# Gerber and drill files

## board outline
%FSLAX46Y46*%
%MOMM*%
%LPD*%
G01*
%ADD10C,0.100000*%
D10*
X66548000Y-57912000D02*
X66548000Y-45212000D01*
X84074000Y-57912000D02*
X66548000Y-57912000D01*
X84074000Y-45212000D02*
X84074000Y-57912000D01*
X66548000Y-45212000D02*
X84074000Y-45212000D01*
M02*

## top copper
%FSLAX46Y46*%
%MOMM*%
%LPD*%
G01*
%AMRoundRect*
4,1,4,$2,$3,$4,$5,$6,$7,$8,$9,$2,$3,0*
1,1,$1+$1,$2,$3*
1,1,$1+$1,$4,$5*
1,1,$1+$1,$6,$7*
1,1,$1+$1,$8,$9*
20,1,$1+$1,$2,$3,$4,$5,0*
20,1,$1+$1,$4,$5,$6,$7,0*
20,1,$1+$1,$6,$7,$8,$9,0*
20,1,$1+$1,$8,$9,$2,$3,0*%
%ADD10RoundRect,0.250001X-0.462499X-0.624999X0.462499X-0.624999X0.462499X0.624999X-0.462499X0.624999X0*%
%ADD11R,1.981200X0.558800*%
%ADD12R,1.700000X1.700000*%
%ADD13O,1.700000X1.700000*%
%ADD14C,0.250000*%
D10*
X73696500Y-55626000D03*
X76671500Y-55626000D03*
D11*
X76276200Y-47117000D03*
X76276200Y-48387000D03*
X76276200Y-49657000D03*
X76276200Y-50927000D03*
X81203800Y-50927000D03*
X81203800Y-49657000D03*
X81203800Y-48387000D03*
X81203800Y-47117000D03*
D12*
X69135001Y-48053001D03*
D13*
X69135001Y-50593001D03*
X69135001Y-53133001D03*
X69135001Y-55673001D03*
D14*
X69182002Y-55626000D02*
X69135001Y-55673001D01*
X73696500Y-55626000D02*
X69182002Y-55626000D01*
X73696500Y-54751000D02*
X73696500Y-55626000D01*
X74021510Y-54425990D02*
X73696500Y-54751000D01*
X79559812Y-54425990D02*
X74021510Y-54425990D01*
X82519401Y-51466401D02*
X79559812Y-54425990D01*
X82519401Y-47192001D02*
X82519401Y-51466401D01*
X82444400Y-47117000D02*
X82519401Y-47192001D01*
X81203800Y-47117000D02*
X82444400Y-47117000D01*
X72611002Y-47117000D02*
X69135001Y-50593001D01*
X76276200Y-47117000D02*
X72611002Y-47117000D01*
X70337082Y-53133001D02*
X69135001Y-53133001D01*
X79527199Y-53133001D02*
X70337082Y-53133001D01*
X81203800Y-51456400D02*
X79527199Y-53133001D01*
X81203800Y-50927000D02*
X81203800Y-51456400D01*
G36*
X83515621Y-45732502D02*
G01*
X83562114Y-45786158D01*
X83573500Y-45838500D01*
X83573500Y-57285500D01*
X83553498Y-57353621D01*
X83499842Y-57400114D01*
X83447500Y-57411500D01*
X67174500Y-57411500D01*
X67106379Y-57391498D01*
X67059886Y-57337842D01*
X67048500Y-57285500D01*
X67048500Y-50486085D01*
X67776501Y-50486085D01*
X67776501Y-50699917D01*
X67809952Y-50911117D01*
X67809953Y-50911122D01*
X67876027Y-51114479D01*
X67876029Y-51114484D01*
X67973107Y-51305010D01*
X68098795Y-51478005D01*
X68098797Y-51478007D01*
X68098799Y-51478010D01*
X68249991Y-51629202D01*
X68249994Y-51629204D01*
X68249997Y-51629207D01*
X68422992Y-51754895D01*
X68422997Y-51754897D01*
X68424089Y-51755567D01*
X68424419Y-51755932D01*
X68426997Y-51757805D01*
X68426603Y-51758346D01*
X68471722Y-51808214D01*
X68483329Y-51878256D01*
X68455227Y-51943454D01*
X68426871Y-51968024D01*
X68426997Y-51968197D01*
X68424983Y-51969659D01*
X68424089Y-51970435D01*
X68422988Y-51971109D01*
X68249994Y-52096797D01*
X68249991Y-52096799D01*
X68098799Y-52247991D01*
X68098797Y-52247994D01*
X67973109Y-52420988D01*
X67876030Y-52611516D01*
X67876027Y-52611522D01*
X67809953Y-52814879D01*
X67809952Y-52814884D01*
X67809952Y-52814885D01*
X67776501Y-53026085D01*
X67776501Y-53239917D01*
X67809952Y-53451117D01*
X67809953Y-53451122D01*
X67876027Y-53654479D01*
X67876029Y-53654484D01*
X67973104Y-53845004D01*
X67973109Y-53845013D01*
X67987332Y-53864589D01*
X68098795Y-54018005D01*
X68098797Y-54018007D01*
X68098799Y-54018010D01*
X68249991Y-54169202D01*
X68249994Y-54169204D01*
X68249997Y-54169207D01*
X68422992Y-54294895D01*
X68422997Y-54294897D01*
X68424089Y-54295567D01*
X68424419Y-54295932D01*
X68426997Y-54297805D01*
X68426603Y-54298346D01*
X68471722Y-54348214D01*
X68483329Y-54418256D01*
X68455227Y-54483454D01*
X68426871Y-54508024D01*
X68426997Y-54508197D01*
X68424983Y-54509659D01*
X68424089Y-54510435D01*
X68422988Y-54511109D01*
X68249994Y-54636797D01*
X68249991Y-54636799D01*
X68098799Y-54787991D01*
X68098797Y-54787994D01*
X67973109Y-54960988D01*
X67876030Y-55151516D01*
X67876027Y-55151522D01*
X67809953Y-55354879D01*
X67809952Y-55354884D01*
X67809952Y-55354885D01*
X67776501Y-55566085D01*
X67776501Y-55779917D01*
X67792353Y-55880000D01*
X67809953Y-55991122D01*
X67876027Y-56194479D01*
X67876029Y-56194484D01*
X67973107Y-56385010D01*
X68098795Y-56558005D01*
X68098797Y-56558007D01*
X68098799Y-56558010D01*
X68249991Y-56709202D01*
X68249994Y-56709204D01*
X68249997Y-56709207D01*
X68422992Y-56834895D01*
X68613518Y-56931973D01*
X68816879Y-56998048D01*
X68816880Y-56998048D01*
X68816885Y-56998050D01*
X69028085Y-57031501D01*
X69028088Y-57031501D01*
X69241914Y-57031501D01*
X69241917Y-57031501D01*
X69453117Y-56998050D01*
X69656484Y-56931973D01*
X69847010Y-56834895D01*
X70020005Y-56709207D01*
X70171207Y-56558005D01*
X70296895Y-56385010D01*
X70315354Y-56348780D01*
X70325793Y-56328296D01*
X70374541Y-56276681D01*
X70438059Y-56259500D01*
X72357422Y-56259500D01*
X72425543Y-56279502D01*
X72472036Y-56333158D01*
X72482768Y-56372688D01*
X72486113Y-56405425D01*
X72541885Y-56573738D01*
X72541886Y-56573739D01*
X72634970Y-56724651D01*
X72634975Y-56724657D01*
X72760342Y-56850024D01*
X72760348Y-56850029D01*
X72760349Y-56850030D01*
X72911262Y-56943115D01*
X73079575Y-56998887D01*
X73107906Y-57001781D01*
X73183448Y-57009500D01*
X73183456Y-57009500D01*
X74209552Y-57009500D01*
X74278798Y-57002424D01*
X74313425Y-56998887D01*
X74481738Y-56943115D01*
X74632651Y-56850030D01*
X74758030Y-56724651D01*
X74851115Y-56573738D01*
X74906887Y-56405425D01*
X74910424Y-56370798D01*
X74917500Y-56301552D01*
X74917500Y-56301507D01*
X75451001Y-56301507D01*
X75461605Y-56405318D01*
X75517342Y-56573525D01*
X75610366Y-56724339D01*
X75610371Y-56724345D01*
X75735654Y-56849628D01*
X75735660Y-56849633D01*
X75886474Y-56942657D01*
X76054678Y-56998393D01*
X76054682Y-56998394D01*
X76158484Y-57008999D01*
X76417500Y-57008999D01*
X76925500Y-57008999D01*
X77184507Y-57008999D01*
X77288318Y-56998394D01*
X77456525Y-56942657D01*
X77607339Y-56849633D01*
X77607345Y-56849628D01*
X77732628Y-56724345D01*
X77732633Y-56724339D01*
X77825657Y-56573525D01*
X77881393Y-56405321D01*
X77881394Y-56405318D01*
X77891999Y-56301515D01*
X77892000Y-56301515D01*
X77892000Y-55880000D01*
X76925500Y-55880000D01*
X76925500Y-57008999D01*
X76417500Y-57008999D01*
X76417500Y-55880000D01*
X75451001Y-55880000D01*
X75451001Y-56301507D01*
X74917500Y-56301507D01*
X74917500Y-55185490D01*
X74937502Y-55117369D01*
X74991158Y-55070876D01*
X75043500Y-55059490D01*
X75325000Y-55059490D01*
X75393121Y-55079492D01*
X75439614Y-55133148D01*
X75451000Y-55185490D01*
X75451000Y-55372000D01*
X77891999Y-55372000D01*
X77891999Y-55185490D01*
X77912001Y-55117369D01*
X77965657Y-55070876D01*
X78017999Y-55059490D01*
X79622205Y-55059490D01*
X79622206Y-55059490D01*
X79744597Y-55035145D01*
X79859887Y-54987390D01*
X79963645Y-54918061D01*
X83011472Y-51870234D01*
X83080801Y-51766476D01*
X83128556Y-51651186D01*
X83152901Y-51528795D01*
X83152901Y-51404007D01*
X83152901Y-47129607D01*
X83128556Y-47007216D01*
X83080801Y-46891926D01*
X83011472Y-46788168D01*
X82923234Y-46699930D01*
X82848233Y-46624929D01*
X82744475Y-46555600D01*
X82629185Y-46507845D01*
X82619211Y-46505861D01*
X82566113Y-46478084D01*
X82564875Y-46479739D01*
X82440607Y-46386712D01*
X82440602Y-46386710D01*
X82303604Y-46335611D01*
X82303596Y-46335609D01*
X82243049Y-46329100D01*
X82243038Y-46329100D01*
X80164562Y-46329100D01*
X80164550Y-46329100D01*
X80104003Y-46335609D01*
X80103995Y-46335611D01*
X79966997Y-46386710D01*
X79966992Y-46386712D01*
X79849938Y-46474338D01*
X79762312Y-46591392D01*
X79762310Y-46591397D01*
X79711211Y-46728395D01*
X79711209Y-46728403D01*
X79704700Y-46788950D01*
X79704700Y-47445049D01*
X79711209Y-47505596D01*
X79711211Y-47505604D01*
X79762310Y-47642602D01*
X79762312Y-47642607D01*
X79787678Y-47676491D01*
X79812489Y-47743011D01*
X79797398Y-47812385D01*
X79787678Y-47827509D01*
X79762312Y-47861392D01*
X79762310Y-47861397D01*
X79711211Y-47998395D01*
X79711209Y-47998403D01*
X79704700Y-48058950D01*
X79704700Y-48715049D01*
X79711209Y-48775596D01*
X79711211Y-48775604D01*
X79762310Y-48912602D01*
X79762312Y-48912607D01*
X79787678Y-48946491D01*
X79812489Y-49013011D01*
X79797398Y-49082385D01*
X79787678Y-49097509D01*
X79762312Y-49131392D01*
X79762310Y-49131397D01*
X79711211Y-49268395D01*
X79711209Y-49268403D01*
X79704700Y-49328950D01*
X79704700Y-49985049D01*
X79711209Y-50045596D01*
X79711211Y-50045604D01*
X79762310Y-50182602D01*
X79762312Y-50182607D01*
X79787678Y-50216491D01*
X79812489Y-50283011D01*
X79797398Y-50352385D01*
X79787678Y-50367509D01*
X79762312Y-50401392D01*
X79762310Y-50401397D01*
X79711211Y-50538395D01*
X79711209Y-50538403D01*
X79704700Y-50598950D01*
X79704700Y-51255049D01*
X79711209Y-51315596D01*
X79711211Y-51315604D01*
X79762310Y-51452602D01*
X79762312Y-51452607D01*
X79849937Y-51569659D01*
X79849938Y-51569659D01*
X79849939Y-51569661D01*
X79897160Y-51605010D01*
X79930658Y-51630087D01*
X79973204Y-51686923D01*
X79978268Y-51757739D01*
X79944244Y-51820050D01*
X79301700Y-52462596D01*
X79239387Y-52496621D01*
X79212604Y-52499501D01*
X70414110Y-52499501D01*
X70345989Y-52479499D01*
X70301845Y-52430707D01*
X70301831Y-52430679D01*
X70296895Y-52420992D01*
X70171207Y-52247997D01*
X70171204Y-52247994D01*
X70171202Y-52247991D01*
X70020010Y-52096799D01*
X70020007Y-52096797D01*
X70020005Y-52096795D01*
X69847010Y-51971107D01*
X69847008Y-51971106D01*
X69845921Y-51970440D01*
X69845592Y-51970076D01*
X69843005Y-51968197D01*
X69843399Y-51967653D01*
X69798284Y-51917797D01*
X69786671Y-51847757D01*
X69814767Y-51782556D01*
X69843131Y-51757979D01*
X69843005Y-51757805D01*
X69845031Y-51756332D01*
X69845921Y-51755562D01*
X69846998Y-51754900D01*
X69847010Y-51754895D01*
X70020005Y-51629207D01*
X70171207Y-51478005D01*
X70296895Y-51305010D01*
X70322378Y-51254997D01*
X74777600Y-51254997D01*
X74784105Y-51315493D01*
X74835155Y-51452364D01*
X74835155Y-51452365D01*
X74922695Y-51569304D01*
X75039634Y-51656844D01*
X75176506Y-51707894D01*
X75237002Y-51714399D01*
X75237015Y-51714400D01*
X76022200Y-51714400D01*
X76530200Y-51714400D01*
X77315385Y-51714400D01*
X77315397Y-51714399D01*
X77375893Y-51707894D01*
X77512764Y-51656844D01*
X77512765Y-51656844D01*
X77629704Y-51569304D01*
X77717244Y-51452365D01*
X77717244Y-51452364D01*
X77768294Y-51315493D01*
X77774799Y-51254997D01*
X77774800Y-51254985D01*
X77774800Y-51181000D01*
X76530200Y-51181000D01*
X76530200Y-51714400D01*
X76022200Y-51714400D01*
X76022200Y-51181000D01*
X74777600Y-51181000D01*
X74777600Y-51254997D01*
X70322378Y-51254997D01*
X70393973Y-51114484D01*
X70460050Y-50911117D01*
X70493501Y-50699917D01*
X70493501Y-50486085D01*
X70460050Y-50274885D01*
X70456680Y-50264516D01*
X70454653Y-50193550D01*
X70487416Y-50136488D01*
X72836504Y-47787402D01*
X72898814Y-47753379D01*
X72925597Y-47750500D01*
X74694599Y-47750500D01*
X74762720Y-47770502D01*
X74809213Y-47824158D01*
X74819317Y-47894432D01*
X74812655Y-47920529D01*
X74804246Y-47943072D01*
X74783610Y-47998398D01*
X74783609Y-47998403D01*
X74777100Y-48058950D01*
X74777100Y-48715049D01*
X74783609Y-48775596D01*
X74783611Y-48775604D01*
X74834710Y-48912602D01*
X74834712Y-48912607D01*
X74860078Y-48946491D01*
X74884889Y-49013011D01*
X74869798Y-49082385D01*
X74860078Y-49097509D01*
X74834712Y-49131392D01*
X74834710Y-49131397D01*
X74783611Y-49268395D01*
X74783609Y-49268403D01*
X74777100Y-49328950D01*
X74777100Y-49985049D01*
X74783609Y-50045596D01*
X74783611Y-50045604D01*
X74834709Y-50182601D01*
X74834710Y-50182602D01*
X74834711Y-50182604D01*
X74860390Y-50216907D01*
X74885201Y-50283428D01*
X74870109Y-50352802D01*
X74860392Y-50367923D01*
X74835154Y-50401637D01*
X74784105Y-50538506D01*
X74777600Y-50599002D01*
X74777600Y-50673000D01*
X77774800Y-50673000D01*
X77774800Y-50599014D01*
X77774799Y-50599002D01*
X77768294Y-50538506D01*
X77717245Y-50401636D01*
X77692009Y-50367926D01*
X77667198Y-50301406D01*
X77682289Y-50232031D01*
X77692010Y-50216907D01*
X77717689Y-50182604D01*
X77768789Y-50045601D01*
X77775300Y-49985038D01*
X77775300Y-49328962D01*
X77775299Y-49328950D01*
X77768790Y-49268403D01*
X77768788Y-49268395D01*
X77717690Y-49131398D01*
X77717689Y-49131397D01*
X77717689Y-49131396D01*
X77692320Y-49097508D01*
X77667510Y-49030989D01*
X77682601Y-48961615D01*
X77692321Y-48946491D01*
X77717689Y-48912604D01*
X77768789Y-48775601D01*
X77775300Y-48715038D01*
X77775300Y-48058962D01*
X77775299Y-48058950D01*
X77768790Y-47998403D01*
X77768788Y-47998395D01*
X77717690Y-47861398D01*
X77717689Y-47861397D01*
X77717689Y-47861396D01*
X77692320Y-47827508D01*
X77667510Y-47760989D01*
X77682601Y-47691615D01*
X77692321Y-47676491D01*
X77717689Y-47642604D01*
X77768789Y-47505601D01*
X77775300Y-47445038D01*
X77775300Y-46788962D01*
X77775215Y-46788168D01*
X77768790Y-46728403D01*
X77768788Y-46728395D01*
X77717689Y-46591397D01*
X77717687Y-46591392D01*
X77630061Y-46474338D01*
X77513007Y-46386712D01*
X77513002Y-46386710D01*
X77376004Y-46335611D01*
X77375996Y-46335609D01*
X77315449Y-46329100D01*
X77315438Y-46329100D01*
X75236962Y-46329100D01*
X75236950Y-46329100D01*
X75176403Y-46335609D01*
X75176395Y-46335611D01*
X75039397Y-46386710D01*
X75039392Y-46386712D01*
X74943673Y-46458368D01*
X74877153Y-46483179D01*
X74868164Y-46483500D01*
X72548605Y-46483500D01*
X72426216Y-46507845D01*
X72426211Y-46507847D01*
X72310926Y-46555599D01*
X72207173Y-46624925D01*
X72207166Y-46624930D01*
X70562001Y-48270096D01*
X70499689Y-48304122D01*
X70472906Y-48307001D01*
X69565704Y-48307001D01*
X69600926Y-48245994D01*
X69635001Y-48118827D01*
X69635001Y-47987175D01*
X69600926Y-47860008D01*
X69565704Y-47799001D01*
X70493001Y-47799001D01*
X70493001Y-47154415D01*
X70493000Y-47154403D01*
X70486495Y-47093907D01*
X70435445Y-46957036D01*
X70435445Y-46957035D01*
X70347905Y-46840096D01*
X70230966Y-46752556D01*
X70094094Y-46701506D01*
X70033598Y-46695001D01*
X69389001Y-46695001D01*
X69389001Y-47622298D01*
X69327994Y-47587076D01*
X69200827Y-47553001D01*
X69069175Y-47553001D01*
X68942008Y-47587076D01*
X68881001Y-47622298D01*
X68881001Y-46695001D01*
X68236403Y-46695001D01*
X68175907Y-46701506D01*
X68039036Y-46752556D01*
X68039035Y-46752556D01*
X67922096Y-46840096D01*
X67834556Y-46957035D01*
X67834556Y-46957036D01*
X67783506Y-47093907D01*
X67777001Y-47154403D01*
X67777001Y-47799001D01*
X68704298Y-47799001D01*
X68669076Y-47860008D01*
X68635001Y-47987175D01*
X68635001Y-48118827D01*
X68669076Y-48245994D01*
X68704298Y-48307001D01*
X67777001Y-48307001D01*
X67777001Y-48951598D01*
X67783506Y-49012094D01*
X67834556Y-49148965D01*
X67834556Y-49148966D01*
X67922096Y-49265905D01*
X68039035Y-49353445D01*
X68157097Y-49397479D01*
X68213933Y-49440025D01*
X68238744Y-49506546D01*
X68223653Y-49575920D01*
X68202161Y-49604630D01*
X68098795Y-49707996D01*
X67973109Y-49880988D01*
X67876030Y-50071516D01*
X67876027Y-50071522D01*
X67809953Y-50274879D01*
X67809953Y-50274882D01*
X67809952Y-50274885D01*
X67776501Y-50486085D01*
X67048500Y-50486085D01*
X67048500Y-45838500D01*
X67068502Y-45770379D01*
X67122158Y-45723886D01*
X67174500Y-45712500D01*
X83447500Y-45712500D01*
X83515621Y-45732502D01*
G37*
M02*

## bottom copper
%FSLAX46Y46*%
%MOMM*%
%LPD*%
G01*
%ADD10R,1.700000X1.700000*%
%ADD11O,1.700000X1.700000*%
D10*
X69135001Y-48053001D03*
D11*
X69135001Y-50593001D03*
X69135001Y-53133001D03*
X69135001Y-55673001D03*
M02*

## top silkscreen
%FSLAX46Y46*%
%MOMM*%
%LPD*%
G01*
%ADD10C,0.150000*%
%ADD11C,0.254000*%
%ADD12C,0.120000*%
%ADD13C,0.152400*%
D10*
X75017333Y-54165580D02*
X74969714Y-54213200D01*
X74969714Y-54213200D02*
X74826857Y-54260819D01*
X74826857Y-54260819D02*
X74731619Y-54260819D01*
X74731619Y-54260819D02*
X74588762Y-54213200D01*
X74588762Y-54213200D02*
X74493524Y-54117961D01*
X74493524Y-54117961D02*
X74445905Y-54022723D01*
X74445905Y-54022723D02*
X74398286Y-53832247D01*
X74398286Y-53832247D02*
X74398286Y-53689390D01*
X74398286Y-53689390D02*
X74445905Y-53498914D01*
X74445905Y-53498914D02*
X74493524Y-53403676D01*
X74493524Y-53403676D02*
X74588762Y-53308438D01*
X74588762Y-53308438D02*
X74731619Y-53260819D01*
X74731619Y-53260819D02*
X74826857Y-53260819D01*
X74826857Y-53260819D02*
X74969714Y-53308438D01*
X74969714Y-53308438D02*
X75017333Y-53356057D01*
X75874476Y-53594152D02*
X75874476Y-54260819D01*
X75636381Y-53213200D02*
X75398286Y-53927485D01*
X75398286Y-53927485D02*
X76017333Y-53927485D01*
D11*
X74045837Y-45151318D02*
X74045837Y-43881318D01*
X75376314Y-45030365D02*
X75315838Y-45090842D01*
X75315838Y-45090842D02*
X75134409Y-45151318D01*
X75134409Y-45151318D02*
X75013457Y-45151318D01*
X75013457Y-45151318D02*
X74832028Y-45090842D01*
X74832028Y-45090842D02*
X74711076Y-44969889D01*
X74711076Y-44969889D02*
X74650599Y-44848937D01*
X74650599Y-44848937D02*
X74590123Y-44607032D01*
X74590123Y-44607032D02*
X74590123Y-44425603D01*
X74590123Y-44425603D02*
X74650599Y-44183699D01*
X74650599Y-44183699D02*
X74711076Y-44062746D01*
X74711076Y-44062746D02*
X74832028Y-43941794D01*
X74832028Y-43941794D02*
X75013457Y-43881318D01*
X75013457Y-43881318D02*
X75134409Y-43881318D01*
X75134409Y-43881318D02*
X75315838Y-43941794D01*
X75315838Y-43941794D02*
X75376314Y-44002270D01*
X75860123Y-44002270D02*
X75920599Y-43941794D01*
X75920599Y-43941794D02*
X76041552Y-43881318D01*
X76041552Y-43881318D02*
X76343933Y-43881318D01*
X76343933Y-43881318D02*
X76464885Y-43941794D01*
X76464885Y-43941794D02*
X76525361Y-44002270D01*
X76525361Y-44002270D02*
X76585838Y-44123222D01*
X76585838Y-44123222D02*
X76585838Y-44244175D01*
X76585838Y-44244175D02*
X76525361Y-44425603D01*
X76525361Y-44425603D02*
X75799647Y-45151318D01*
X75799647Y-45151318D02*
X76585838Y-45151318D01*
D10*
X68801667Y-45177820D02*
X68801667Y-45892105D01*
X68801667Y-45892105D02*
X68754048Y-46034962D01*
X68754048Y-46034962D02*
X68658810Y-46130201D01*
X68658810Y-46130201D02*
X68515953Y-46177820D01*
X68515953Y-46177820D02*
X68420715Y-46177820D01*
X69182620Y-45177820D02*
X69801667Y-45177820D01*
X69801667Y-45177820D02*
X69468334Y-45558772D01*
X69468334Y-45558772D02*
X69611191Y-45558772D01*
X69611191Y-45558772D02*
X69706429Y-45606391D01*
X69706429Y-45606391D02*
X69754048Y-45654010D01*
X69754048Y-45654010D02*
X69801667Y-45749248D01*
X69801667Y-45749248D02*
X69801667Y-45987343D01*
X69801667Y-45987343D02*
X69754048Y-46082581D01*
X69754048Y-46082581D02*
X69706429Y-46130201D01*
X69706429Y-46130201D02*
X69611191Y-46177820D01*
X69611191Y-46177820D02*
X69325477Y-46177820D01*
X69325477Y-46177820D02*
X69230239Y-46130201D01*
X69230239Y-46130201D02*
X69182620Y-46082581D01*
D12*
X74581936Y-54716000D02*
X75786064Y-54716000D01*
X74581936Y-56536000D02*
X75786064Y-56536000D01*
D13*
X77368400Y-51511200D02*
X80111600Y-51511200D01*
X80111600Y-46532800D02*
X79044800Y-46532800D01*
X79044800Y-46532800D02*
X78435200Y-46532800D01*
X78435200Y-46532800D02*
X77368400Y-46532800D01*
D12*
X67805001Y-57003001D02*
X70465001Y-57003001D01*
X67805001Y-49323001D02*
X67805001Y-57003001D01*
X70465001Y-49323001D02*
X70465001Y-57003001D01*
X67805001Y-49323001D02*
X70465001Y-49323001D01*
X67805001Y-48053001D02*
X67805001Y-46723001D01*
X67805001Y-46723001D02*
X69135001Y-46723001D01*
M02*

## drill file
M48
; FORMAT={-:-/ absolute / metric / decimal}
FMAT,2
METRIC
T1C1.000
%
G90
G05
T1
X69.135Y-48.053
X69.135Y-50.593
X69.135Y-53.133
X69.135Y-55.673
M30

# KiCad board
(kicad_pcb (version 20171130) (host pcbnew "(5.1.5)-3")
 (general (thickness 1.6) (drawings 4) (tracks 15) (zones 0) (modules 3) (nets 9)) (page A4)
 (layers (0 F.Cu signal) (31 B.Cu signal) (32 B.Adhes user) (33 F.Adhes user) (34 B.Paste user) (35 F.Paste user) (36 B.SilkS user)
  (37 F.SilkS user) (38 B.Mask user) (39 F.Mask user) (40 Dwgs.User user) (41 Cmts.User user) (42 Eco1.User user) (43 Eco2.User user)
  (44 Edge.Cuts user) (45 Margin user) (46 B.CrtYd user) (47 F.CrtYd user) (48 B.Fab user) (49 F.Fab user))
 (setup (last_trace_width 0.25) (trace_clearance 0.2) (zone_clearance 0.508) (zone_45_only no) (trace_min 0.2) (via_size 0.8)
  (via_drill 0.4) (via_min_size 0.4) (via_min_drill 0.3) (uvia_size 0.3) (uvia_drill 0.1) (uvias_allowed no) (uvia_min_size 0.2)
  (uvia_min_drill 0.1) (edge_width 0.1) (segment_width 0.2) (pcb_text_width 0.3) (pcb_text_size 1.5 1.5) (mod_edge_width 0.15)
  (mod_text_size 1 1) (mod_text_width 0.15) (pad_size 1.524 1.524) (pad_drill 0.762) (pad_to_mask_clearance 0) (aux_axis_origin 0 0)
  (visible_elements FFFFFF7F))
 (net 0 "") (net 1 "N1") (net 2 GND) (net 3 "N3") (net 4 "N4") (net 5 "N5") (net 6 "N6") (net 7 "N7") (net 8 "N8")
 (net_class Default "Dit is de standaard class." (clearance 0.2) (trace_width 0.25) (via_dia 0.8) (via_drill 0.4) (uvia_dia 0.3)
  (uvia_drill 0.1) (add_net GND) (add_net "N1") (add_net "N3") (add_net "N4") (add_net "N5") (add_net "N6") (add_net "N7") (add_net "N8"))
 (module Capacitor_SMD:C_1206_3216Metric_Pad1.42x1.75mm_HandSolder (layer F.Cu) (at 75.184 55.626)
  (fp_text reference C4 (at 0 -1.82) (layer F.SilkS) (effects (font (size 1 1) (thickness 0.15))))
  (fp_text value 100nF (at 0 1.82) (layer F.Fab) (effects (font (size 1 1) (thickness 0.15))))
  (fp_line (start -0.602064 -0.91) (end 0.602064 -0.91) (layer F.SilkS) (width 0.12))
  (fp_line (start -0.602064 0.91) (end 0.602064 0.91) (layer F.SilkS) (width 0.12))
  (pad 1 smd roundrect (at -1.4875 0) (size 1.425 1.75) (layers F.Cu F.Paste F.Mask) (roundrect_rratio 0.175439) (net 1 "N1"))
  (pad 2 smd roundrect (at 1.4875 0) (size 1.425 1.75) (layers F.Cu F.Paste F.Mask) (roundrect_rratio 0.175439) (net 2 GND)))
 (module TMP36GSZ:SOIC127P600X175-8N (layer F.Cu) (at 78.74 49.022)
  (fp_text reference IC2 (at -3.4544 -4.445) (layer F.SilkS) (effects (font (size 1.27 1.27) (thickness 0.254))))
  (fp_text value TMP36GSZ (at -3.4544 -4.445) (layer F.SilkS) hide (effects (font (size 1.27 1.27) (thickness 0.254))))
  (fp_line (start -1.3716 2.4892) (end 1.3716 2.4892) (layer F.SilkS) (width 0.1524))
  (fp_line (start 1.3716 -2.4892) (end 0.3048 -2.4892) (layer F.SilkS) (width 0.1524))
  (fp_line (start 0.3048 -2.4892) (end -0.3048 -2.4892) (layer F.SilkS) (width 0.1524))
  (fp_line (start -0.3048 -2.4892) (end -1.3716 -2.4892) (layer F.SilkS) (width 0.1524))
  (pad 1 smd rect (at -2.4638 -1.905 90) (size 0.5588 1.9812) (layers F.Cu F.Paste F.Mask) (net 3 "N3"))
  (pad 2 smd rect (at -2.4638 -0.635 90) (size 0.5588 1.9812) (layers F.Cu F.Paste F.Mask) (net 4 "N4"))
  (pad 3 smd rect (at -2.4638 0.635 90) (size 0.5588 1.9812) (layers F.Cu F.Paste F.Mask) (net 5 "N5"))
  (pad 4 smd rect (at -2.4638 1.905 90) (size 0.5588 1.9812) (layers F.Cu F.Paste F.Mask) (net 2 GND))
  (pad 5 smd rect (at 2.4638 1.905 90) (size 0.5588 1.9812) (layers F.Cu F.Paste F.Mask) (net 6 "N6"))
  (pad 6 smd rect (at 2.4638 0.635 90) (size 0.5588 1.9812) (layers F.Cu F.Paste F.Mask) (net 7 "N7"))
  (pad 7 smd rect (at 2.4638 -0.635 90) (size 0.5588 1.9812) (layers F.Cu F.Paste F.Mask) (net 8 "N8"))
  (pad 8 smd rect (at 2.4638 -1.905 90) (size 0.5588 1.9812) (layers F.Cu F.Paste F.Mask) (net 1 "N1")))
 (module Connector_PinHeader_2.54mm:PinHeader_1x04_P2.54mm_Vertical (layer F.Cu) (at 69.135001 48.053001)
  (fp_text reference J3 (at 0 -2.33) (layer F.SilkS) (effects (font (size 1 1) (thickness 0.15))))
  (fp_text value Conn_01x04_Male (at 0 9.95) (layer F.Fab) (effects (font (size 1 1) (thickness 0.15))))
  (fp_line (start -1.33 8.95) (end 1.33 8.95) (layer F.SilkS) (width 0.12))
  (fp_line (start -1.33 1.27) (end -1.33 8.95) (layer F.SilkS) (width 0.12))
  (fp_line (start 1.33 1.27) (end 1.33 8.95) (layer F.SilkS) (width 0.12))
  (fp_line (start -1.33 1.27) (end 1.33 1.27) (layer F.SilkS) (width 0.12))
  (fp_line (start -1.33 0) (end -1.33 -1.33) (layer F.SilkS) (width 0.12))
  (fp_line (start -1.33 -1.33) (end 0 -1.33) (layer F.SilkS) (width 0.12))
  (pad 1 thru_hole rect (at 0 0) (size 1.7 1.7) (drill 1) (layers *.Cu *.Mask) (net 2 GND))
  (pad 2 thru_hole oval (at 0 2.54) (size 1.7 1.7) (drill 1) (layers *.Cu *.Mask) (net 3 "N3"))
  (pad 3 thru_hole oval (at 0 5.08) (size 1.7 1.7) (drill 1) (layers *.Cu *.Mask) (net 6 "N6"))
  (pad 4 thru_hole oval (at 0 7.62) (size 1.7 1.7) (drill 1) (layers *.Cu *.Mask) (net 1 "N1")))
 (gr_line (start 66.548 57.912) (end 66.548 45.212) (layer Edge.Cuts) (width 0.1))
 (gr_line (start 84.074 57.912) (end 66.548 57.912) (layer Edge.Cuts) (width 0.1))
 (gr_line (start 84.074 45.212) (end 84.074 57.912) (layer Edge.Cuts) (width 0.1))
 (gr_line (start 66.548 45.212) (end 84.074 45.212) (layer Edge.Cuts) (width 0.1))
 (segment (start 69.182002 55.626) (end 69.135001 55.673001) (width 0.25) (layer F.Cu) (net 1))
 (segment (start 73.6965 55.626) (end 69.182002 55.626) (width 0.25) (layer F.Cu) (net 1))
 (segment (start 73.6965 54.751) (end 73.6965 55.626) (width 0.25) (layer F.Cu) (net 1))
 (segment (start 74.02151 54.42599) (end 73.6965 54.751) (width 0.25) (layer F.Cu) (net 1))
 (segment (start 79.559812 54.42599) (end 74.02151 54.42599) (width 0.25) (layer F.Cu) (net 1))
 (segment (start 82.519401 51.466401) (end 79.559812 54.42599) (width 0.25) (layer F.Cu) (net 1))
 (segment (start 82.519401 47.192001) (end 82.519401 51.466401) (width 0.25) (layer F.Cu) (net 1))
 (segment (start 82.4444 47.117) (end 82.519401 47.192001) (width 0.25) (layer F.Cu) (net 1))
 (segment (start 81.2038 47.117) (end 82.4444 47.117) (width 0.25) (layer F.Cu) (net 1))
 (segment (start 72.611002 47.117) (end 69.135001 50.593001) (width 0.25) (layer F.Cu) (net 3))
 (segment (start 76.2762 47.117) (end 72.611002 47.117) (width 0.25) (layer F.Cu) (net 3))
 (segment (start 70.337082 53.133001) (end 69.135001 53.133001) (width 0.25) (layer F.Cu) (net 6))
 (segment (start 79.527199 53.133001) (end 70.337082 53.133001) (width 0.25) (layer F.Cu) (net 6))
 (segment (start 81.2038 51.4564) (end 79.527199 53.133001) (width 0.25) (layer F.Cu) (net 6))
 (segment (start 81.2038 50.927) (end 81.2038 51.4564) (width 0.25) (layer F.Cu) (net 6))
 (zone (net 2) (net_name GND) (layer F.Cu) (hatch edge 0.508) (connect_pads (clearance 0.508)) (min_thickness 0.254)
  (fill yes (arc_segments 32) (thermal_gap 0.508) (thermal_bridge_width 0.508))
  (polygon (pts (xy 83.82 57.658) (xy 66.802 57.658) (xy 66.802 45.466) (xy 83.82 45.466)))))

